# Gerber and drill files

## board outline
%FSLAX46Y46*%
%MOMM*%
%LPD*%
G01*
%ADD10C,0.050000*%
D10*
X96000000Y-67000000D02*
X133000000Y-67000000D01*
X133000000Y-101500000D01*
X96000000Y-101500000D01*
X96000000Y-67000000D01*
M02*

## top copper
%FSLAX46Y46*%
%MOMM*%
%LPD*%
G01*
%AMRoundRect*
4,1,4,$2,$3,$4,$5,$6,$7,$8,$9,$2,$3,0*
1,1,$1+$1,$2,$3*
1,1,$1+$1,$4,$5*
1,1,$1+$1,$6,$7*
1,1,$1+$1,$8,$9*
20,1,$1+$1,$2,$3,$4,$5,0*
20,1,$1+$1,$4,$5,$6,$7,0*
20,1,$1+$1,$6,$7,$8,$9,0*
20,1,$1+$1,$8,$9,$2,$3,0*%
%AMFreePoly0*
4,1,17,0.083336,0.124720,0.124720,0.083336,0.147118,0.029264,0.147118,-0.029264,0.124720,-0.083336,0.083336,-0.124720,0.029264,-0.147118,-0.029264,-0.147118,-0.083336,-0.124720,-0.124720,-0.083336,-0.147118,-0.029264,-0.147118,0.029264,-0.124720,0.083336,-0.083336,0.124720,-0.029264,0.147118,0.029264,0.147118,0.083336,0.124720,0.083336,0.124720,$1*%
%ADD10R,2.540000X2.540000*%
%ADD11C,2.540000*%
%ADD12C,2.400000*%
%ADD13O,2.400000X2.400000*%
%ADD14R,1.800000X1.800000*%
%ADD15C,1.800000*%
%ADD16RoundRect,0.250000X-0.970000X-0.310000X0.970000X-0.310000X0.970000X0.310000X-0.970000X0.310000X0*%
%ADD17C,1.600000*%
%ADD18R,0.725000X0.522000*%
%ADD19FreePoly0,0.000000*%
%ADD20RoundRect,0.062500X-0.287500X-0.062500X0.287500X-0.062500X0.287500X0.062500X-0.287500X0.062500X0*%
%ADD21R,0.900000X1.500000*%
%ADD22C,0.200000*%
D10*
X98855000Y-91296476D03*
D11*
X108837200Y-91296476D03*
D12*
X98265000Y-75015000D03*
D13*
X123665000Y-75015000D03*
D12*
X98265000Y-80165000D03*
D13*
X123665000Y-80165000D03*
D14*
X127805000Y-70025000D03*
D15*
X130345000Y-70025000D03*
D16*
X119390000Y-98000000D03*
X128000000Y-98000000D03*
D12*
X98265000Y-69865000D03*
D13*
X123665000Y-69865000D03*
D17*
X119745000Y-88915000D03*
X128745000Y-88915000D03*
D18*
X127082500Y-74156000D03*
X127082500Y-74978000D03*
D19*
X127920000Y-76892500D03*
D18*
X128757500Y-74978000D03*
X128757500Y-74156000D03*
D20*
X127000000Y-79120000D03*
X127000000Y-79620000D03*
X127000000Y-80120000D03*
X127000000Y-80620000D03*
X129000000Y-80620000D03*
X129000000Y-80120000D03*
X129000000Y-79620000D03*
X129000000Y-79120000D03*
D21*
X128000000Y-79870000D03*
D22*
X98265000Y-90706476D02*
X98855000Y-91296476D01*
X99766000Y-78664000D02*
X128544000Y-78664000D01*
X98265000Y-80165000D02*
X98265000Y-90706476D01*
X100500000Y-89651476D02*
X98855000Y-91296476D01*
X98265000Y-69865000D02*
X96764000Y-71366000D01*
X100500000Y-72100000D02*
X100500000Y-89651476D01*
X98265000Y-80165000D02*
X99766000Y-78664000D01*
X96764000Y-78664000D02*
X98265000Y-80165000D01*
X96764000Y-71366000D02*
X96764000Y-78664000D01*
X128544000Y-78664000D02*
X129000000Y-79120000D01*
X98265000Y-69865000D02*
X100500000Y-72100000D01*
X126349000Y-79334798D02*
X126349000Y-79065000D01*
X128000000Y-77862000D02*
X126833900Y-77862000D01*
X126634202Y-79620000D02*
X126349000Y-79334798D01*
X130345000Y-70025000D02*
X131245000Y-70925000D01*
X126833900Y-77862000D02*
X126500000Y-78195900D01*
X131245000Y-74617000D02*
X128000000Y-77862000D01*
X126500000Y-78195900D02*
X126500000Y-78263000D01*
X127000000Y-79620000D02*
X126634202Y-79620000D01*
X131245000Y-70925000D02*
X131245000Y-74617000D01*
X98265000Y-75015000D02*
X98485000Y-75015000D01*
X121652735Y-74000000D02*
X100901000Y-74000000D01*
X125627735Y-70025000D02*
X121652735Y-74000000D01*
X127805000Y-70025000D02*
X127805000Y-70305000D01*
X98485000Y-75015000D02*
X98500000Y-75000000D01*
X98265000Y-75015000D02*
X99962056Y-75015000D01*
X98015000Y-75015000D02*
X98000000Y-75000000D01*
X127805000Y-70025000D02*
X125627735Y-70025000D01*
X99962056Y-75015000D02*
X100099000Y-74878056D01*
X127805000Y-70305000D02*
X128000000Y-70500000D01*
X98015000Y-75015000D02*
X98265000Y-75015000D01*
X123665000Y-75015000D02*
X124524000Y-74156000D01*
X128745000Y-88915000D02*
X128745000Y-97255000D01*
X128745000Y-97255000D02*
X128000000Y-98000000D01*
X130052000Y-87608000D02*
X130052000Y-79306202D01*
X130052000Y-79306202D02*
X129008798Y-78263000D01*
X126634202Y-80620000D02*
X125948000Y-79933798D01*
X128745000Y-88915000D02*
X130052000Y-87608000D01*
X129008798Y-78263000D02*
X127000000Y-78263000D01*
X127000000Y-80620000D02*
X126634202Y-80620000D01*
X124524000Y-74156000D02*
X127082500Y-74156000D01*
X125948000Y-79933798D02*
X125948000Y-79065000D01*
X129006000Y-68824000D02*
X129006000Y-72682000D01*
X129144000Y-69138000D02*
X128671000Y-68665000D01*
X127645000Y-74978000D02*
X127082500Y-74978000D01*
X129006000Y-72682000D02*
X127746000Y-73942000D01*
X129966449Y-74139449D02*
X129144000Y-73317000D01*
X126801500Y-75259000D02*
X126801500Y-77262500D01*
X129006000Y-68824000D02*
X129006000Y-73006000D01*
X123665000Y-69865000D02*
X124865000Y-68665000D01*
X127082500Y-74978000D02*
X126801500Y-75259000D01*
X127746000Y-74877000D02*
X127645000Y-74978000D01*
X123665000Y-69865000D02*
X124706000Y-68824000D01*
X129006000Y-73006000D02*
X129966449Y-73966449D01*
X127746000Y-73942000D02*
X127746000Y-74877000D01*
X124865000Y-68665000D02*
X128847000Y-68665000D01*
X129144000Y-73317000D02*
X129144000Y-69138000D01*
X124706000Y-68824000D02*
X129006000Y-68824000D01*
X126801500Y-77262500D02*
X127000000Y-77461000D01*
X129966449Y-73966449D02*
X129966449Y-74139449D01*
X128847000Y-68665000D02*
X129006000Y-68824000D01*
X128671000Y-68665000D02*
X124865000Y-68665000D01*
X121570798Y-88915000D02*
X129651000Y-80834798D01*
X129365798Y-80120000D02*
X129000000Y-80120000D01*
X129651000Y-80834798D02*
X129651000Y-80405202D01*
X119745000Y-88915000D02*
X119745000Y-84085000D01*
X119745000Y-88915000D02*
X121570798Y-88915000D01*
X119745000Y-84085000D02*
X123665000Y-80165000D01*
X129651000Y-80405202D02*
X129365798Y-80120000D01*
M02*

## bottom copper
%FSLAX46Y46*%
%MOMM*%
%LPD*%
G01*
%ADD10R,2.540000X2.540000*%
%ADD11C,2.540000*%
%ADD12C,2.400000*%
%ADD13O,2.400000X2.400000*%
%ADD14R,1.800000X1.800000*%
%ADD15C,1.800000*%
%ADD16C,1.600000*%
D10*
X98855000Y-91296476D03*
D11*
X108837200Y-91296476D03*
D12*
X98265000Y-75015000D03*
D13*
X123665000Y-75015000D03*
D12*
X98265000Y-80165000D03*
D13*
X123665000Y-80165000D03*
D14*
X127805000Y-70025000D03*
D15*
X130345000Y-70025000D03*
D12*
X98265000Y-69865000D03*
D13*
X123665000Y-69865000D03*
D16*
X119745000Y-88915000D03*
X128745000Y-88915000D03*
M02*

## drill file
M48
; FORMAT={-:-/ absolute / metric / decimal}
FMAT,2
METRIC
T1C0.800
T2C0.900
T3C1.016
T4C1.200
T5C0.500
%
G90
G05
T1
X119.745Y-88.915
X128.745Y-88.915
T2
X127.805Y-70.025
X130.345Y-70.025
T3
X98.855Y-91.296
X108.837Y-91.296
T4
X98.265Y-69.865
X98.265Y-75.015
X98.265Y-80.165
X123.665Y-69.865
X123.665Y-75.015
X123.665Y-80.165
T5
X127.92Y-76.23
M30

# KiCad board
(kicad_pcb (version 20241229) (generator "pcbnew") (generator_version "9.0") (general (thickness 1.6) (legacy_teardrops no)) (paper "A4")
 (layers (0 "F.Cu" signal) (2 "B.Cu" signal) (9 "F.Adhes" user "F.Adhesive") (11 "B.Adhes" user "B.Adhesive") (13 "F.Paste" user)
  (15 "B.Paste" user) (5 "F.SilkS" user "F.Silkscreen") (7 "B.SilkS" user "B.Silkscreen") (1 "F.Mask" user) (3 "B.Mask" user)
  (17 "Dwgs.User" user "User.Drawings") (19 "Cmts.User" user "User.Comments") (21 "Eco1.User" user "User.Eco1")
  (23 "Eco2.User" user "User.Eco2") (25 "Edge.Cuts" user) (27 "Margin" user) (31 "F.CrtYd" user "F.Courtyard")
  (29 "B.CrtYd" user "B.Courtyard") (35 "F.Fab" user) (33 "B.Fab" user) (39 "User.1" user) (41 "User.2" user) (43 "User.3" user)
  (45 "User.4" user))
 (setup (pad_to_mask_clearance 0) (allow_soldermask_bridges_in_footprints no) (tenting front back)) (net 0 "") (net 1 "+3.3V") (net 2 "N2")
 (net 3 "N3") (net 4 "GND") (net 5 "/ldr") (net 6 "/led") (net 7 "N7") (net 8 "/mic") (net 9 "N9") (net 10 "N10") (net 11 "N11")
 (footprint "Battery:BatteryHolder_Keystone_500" (layer "F.Cu") (at 98.855 91.296476)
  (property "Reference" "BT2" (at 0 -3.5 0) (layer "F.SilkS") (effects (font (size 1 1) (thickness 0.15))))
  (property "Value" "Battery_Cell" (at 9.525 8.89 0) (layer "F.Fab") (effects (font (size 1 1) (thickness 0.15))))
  (pad "1" thru_hole rect (at 0 0) (size 2.54 2.54) (drill 1.016) (layers "*.Cu" "*.Mask") (remove_unused_layers no) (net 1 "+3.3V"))
  (pad "2" thru_hole circle (at 9.9822 0) (size 2.54 2.54) (drill 1.016) (layers "*.Cu" "*.Mask") (remove_unused_layers no) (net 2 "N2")))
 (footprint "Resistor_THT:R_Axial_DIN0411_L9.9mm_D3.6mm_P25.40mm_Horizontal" (layer "F.Cu") (at 98.265 75.015)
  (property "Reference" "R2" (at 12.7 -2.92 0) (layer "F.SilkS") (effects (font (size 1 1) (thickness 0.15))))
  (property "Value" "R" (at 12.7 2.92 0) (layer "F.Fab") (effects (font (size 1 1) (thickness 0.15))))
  (pad "1" thru_hole circle (at 0 0) (size 2.4 2.4) (drill 1.2) (layers "*.Cu" "*.Mask") (remove_unused_layers no) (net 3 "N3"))
  (pad "2" thru_hole oval (at 25.4 0) (size 2.4 2.4) (drill 1.2) (layers "*.Cu" "*.Mask") (remove_unused_layers no) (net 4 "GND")))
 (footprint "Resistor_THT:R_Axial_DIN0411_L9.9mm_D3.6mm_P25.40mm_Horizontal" (layer "F.Cu") (at 98.265 80.165)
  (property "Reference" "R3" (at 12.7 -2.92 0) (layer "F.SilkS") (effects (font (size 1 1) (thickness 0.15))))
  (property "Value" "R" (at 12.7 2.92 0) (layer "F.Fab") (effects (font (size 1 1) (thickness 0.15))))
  (pad "1" thru_hole circle (at 0 0) (size 2.4 2.4) (drill 1.2) (layers "*.Cu" "*.Mask") (remove_unused_layers no) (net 1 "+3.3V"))
  (pad "2" thru_hole oval (at 25.4 0) (size 2.4 2.4) (drill 1.2) (layers "*.Cu" "*.Mask") (remove_unused_layers no) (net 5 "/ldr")))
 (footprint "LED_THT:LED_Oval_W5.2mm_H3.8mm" (layer "F.Cu") (at 127.805 70.025)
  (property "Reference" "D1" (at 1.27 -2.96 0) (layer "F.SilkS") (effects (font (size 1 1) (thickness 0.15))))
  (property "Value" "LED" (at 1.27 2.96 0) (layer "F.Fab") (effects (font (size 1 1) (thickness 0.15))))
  (pad "1" thru_hole rect (at 0 0) (size 1.8 1.8) (drill 0.9) (layers "*.Cu" "*.Mask") (remove_unused_layers no) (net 3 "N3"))
  (pad "2" thru_hole circle (at 2.54 0) (size 1.8 1.8) (drill 0.9) (layers "*.Cu" "*.Mask") (remove_unused_layers no) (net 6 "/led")))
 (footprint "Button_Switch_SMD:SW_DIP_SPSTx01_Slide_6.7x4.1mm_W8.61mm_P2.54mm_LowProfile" (layer "F.Cu") (at 123.695 98)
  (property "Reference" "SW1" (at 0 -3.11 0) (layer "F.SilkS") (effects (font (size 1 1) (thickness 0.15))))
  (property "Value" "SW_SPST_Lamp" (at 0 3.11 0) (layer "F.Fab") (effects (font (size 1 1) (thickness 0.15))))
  (pad "1" smd roundrect (at -4.305 0) (size 2.44 1.12) (layers "F.Cu" "F.Mask" "F.Paste") (roundrect_rratio 0.223214) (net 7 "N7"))
  (pad "2" smd roundrect (at 4.305 0) (size 2.44 1.12) (layers "F.Cu" "F.Mask" "F.Paste") (roundrect_rratio 0.223214) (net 4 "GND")))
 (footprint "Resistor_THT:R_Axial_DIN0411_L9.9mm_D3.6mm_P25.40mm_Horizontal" (layer "F.Cu") (at 98.265 69.865)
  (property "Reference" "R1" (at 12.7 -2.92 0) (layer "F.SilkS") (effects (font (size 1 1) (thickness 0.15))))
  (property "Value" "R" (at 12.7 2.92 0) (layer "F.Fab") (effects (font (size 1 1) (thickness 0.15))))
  (pad "1" thru_hole circle (at 0 0) (size 2.4 2.4) (drill 1.2) (layers "*.Cu" "*.Mask") (remove_unused_layers no) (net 1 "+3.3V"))
  (pad "2" thru_hole oval (at 25.4 0) (size 2.4 2.4) (drill 1.2) (layers "*.Cu" "*.Mask") (remove_unused_layers no) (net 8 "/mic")))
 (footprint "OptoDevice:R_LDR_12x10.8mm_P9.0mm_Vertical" (layer "F.Cu") (at 119.745 88.915)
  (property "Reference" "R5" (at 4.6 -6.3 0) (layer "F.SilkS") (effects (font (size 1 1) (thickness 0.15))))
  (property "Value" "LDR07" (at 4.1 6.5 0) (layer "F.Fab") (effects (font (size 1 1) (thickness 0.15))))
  (pad "1" thru_hole circle (at 0 0) (size 1.6 1.6) (drill 0.8) (layers "*.Cu" "*.Mask") (remove_unused_layers no) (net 5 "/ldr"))
  (pad "2" thru_hole circle (at 9 0) (size 1.6 1.6) (drill 0.8) (layers "*.Cu" "*.Mask") (remove_unused_layers no) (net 4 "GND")))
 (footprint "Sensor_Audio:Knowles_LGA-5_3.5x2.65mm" (layer "F.Cu") (at 127.92 75.46)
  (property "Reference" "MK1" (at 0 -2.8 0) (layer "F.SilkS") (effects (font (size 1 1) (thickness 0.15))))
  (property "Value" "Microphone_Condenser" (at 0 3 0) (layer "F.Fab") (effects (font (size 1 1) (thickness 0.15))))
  (pad "" np_thru_hole circle (at 0 0.77) (size 0.5 0.5) (drill 0.5) (layers "*.Cu" "*.Mask"))
  (pad "1" smd rect (at -0.8375 -1.304) (size 0.725 0.522) (layers "F.Cu" "F.Mask" "F.Paste") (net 4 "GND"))
  (pad "2" smd rect (at -0.8375 -0.482) (size 0.725 0.522) (layers "F.Cu" "F.Mask" "F.Paste") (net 8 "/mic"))
  (pad "3" smd custom (at 0 1.4325) (size 0.3 0.3) (layers "F.Cu" "F.Mask") (zone_connect 0) (options (clearance outline) (anchor circle))
   (primitives))
  (pad "4" smd rect (at 0.8375 -0.482) (size 0.725 0.522) (layers "F.Cu" "F.Mask" "F.Paste"))
  (pad "5" smd rect (at 0.8375 -1.304) (size 0.725 0.522) (layers "F.Cu" "F.Mask" "F.Paste")))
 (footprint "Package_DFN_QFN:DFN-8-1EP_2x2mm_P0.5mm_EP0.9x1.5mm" (layer "F.Cu") (at 128 79.87)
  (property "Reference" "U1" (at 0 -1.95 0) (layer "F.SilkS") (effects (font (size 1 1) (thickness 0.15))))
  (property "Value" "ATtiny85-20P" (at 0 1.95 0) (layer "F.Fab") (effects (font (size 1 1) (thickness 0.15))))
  (pad "" smd roundrect (at -0.225 -0.375) (size 0.36 0.6) (layers "F.Paste") (roundrect_rratio 0.25))
  (pad "" smd roundrect (at -0.225 0.375) (size 0.36 0.6) (layers "F.Paste") (roundrect_rratio 0.25))
  (pad "" smd roundrect (at 0.225 -0.375) (size 0.36 0.6) (layers "F.Paste") (roundrect_rratio 0.25))
  (pad "" smd roundrect (at 0.225 0.375) (size 0.36 0.6) (layers "F.Paste") (roundrect_rratio 0.25))
  (pad "1" smd roundrect (at -1 -0.75) (size 0.7 0.25) (layers "F.Cu" "F.Mask" "F.Paste") (roundrect_rratio 0.25) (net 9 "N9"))
  (pad "2" smd roundrect (at -1 -0.25) (size 0.7 0.25) (layers "F.Cu" "F.Mask" "F.Paste") (roundrect_rratio 0.25) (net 6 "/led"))
  (pad "3" smd roundrect (at -1 0.25) (size 0.7 0.25) (layers "F.Cu" "F.Mask" "F.Paste") (roundrect_rratio 0.25) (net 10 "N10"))
  (pad "4" smd roundrect (at -1 0.75) (size 0.7 0.25) (layers "F.Cu" "F.Mask" "F.Paste") (roundrect_rratio 0.25) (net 4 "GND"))
  (pad "5" smd roundrect (at 1 0.75) (size 0.7 0.25) (layers "F.Cu" "F.Mask" "F.Paste") (roundrect_rratio 0.25) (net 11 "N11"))
  (pad "6" smd roundrect (at 1 0.25) (size 0.7 0.25) (layers "F.Cu" "F.Mask" "F.Paste") (roundrect_rratio 0.25) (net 5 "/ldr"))
  (pad "7" smd roundrect (at 1 -0.25) (size 0.7 0.25) (layers "F.Cu" "F.Mask" "F.Paste") (roundrect_rratio 0.25) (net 8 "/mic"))
  (pad "8" smd roundrect (at 1 -0.75) (size 0.7 0.25) (layers "F.Cu" "F.Mask" "F.Paste") (roundrect_rratio 0.25) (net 1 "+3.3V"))
  (pad "9" smd rect (at 0 0) (size 0.9 1.5) (layers "F.Cu" "F.Mask") (zone_connect 2)))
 (gr_rect (start 96 67) (end 133 101.5) (stroke (width 0.05) (type default)) (fill no) (layer "Edge.Cuts"))
 (segment (start 98.265 90.706476) (end 98.855 91.296476) (width 0.2) (layer "F.Cu") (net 1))
 (segment (start 99.766 78.664) (end 128.544 78.664) (width 0.2) (layer "F.Cu") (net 1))
 (segment (start 98.265 80.165) (end 98.265 90.706476) (width 0.2) (layer "F.Cu") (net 1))
 (segment (start 100.5 89.651476) (end 98.855 91.296476) (width 0.2) (layer "F.Cu") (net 1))
 (segment (start 98.265 69.865) (end 96.764 71.366) (width 0.2) (layer "F.Cu") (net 1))
 (segment (start 100.5 72.1) (end 100.5 89.651476) (width 0.2) (layer "F.Cu") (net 1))
 (segment (start 98.265 80.165) (end 99.766 78.664) (width 0.2) (layer "F.Cu") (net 1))
 (segment (start 96.764 78.664) (end 98.265 80.165) (width 0.2) (layer "F.Cu") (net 1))
 (segment (start 96.764 71.366) (end 96.764 78.664) (width 0.2) (layer "F.Cu") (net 1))
 (segment (start 128.544 78.664) (end 129 79.12) (width 0.2) (layer "F.Cu") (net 1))
 (segment (start 98.265 69.865) (end 100.5 72.1) (width 0.2) (layer "F.Cu") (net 1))
 (segment (start 126.349 79.334798) (end 126.349 79.065) (width 0.2) (layer "F.Cu") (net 6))
 (segment (start 128 77.862) (end 126.8339 77.862) (width 0.2) (layer "F.Cu") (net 6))
 (segment (start 126.634202 79.62) (end 126.349 79.334798) (width 0.2) (layer "F.Cu") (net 6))
 (segment (start 130.345 70.025) (end 131.245 70.925) (width 0.2) (layer "F.Cu") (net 6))
 (segment (start 126.8339 77.862) (end 126.5 78.1959) (width 0.2) (layer "F.Cu") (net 6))
 (segment (start 131.245 74.617) (end 128 77.862) (width 0.2) (layer "F.Cu") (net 6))
 (segment (start 126.5 78.1959) (end 126.5 78.263) (width 0.2) (layer "F.Cu") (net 6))
 (segment (start 127 79.62) (end 126.634202 79.62) (width 0.2) (layer "F.Cu") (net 6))
 (segment (start 131.245 70.925) (end 131.245 74.617) (width 0.2) (layer "F.Cu") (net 6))
 (segment (start 98.265 75.015) (end 98.485 75.015) (width 0.2) (layer "F.Cu") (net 3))
 (segment (start 121.652735 74) (end 100.901 74) (width 0.2) (layer "F.Cu") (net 3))
 (segment (start 125.627735 70.025) (end 121.652735 74) (width 0.2) (layer "F.Cu") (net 3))
 (segment (start 127.805 70.025) (end 127.805 70.305) (width 0.2) (layer "F.Cu") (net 3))
 (segment (start 98.485 75.015) (end 98.5 75) (width 0.2) (layer "F.Cu") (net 3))
 (segment (start 98.265 75.015) (end 99.962056 75.015) (width 0.2) (layer "F.Cu") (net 3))
 (segment (start 98.015 75.015) (end 98 75) (width 0.2) (layer "F.Cu") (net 3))
 (segment (start 127.805 70.025) (end 125.627735 70.025) (width 0.2) (layer "F.Cu") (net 3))
 (segment (start 99.962056 75.015) (end 100.099 74.878056) (width 0.2) (layer "F.Cu") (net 3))
 (segment (start 127.805 70.305) (end 128 70.5) (width 0.2) (layer "F.Cu") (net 3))
 (segment (start 98.015 75.015) (end 98.265 75.015) (width 0.2) (layer "F.Cu") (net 3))
 (segment (start 123.665 75.015) (end 124.524 74.156) (width 0.2) (layer "F.Cu") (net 4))
 (segment (start 128.745 88.915) (end 128.745 97.255) (width 0.2) (layer "F.Cu") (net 4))
 (segment (start 128.745 97.255) (end 128 98) (width 0.2) (layer "F.Cu") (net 4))
 (segment (start 130.052 87.608) (end 130.052 79.306202) (width 0.2) (layer "F.Cu") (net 4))
 (segment (start 130.052 79.306202) (end 129.008798 78.263) (width 0.2) (layer "F.Cu") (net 4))
 (segment (start 126.634202 80.62) (end 125.948 79.933798) (width 0.2) (layer "F.Cu") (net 4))
 (segment (start 128.745 88.915) (end 130.052 87.608) (width 0.2) (layer "F.Cu") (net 4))
 (segment (start 129.008798 78.263) (end 127 78.263) (width 0.2) (layer "F.Cu") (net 4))
 (segment (start 127 80.62) (end 126.634202 80.62) (width 0.2) (layer "F.Cu") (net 4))
 (segment (start 124.524 74.156) (end 127.0825 74.156) (width 0.2) (layer "F.Cu") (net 4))
 (segment (start 125.948 79.933798) (end 125.948 79.065) (width 0.2) (layer "F.Cu") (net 4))
 (segment (start 129.006 68.824) (end 129.006 72.682) (width 0.2) (layer "F.Cu") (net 8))
 (segment (start 129.144 69.138) (end 128.671 68.665) (width 0.2) (layer "F.Cu") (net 8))
 (segment (start 127.645 74.978) (end 127.0825 74.978) (width 0.2) (layer "F.Cu") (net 8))
 (segment (start 129.006 72.682) (end 127.746 73.942) (width 0.2) (layer "F.Cu") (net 8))
 (segment (start 129.966449 74.139449) (end 129.144 73.317) (width 0.2) (layer "F.Cu") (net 8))
 (segment (start 126.8015 75.259) (end 126.8015 77.2625) (width 0.2) (layer "F.Cu") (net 8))
 (segment (start 129.006 68.824) (end 129.006 73.006) (width 0.2) (layer "F.Cu") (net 8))
 (segment (start 123.665 69.865) (end 124.865 68.665) (width 0.2) (layer "F.Cu") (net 8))
 (segment (start 127.0825 74.978) (end 126.8015 75.259) (width 0.2) (layer "F.Cu") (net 8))
 (segment (start 127.746 74.877) (end 127.645 74.978) (width 0.2) (layer "F.Cu") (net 8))
 (segment (start 123.665 69.865) (end 124.706 68.824) (width 0.2) (layer "F.Cu") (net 8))
 (segment (start 129.006 73.006) (end 129.966449 73.966449) (width 0.2) (layer "F.Cu") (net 8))
 (segment (start 127.746 73.942) (end 127.746 74.877) (width 0.2) (layer "F.Cu") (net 8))
 (segment (start 124.865 68.665) (end 128.847 68.665) (width 0.2) (layer "F.Cu") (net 8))
 (segment (start 129.144 73.317) (end 129.144 69.138) (width 0.2) (layer "F.Cu") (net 8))
 (segment (start 124.706 68.824) (end 129.006 68.824) (width 0.2) (layer "F.Cu") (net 8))
 (segment (start 126.8015 77.2625) (end 127 77.461) (width 0.2) (layer "F.Cu") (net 8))
 (segment (start 129.966449 73.966449) (end 129.966449 74.139449) (width 0.2) (layer "F.Cu") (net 8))
 (segment (start 128.847 68.665) (end 129.006 68.824) (width 0.2) (layer "F.Cu") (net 8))
 (segment (start 128.671 68.665) (end 124.865 68.665) (width 0.2) (layer "F.Cu") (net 8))
 (segment (start 121.570798 88.915) (end 129.651 80.834798) (width 0.2) (layer "F.Cu") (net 5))
 (segment (start 129.365798 80.12) (end 129 80.12) (width 0.2) (layer "F.Cu") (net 5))
 (segment (start 129.651 80.834798) (end 129.651 80.405202) (width 0.2) (layer "F.Cu") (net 5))
 (segment (start 119.745 88.915) (end 119.745 84.085) (width 0.2) (layer "F.Cu") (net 5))
 (segment (start 119.745 88.915) (end 121.570798 88.915) (width 0.2) (layer "F.Cu") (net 5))
 (segment (start 119.745 84.085) (end 123.665 80.165) (width 0.2) (layer "F.Cu") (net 5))
 (segment (start 129.651 80.405202) (end 129.365798 80.12) (width 0.2) (layer "F.Cu") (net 5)))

